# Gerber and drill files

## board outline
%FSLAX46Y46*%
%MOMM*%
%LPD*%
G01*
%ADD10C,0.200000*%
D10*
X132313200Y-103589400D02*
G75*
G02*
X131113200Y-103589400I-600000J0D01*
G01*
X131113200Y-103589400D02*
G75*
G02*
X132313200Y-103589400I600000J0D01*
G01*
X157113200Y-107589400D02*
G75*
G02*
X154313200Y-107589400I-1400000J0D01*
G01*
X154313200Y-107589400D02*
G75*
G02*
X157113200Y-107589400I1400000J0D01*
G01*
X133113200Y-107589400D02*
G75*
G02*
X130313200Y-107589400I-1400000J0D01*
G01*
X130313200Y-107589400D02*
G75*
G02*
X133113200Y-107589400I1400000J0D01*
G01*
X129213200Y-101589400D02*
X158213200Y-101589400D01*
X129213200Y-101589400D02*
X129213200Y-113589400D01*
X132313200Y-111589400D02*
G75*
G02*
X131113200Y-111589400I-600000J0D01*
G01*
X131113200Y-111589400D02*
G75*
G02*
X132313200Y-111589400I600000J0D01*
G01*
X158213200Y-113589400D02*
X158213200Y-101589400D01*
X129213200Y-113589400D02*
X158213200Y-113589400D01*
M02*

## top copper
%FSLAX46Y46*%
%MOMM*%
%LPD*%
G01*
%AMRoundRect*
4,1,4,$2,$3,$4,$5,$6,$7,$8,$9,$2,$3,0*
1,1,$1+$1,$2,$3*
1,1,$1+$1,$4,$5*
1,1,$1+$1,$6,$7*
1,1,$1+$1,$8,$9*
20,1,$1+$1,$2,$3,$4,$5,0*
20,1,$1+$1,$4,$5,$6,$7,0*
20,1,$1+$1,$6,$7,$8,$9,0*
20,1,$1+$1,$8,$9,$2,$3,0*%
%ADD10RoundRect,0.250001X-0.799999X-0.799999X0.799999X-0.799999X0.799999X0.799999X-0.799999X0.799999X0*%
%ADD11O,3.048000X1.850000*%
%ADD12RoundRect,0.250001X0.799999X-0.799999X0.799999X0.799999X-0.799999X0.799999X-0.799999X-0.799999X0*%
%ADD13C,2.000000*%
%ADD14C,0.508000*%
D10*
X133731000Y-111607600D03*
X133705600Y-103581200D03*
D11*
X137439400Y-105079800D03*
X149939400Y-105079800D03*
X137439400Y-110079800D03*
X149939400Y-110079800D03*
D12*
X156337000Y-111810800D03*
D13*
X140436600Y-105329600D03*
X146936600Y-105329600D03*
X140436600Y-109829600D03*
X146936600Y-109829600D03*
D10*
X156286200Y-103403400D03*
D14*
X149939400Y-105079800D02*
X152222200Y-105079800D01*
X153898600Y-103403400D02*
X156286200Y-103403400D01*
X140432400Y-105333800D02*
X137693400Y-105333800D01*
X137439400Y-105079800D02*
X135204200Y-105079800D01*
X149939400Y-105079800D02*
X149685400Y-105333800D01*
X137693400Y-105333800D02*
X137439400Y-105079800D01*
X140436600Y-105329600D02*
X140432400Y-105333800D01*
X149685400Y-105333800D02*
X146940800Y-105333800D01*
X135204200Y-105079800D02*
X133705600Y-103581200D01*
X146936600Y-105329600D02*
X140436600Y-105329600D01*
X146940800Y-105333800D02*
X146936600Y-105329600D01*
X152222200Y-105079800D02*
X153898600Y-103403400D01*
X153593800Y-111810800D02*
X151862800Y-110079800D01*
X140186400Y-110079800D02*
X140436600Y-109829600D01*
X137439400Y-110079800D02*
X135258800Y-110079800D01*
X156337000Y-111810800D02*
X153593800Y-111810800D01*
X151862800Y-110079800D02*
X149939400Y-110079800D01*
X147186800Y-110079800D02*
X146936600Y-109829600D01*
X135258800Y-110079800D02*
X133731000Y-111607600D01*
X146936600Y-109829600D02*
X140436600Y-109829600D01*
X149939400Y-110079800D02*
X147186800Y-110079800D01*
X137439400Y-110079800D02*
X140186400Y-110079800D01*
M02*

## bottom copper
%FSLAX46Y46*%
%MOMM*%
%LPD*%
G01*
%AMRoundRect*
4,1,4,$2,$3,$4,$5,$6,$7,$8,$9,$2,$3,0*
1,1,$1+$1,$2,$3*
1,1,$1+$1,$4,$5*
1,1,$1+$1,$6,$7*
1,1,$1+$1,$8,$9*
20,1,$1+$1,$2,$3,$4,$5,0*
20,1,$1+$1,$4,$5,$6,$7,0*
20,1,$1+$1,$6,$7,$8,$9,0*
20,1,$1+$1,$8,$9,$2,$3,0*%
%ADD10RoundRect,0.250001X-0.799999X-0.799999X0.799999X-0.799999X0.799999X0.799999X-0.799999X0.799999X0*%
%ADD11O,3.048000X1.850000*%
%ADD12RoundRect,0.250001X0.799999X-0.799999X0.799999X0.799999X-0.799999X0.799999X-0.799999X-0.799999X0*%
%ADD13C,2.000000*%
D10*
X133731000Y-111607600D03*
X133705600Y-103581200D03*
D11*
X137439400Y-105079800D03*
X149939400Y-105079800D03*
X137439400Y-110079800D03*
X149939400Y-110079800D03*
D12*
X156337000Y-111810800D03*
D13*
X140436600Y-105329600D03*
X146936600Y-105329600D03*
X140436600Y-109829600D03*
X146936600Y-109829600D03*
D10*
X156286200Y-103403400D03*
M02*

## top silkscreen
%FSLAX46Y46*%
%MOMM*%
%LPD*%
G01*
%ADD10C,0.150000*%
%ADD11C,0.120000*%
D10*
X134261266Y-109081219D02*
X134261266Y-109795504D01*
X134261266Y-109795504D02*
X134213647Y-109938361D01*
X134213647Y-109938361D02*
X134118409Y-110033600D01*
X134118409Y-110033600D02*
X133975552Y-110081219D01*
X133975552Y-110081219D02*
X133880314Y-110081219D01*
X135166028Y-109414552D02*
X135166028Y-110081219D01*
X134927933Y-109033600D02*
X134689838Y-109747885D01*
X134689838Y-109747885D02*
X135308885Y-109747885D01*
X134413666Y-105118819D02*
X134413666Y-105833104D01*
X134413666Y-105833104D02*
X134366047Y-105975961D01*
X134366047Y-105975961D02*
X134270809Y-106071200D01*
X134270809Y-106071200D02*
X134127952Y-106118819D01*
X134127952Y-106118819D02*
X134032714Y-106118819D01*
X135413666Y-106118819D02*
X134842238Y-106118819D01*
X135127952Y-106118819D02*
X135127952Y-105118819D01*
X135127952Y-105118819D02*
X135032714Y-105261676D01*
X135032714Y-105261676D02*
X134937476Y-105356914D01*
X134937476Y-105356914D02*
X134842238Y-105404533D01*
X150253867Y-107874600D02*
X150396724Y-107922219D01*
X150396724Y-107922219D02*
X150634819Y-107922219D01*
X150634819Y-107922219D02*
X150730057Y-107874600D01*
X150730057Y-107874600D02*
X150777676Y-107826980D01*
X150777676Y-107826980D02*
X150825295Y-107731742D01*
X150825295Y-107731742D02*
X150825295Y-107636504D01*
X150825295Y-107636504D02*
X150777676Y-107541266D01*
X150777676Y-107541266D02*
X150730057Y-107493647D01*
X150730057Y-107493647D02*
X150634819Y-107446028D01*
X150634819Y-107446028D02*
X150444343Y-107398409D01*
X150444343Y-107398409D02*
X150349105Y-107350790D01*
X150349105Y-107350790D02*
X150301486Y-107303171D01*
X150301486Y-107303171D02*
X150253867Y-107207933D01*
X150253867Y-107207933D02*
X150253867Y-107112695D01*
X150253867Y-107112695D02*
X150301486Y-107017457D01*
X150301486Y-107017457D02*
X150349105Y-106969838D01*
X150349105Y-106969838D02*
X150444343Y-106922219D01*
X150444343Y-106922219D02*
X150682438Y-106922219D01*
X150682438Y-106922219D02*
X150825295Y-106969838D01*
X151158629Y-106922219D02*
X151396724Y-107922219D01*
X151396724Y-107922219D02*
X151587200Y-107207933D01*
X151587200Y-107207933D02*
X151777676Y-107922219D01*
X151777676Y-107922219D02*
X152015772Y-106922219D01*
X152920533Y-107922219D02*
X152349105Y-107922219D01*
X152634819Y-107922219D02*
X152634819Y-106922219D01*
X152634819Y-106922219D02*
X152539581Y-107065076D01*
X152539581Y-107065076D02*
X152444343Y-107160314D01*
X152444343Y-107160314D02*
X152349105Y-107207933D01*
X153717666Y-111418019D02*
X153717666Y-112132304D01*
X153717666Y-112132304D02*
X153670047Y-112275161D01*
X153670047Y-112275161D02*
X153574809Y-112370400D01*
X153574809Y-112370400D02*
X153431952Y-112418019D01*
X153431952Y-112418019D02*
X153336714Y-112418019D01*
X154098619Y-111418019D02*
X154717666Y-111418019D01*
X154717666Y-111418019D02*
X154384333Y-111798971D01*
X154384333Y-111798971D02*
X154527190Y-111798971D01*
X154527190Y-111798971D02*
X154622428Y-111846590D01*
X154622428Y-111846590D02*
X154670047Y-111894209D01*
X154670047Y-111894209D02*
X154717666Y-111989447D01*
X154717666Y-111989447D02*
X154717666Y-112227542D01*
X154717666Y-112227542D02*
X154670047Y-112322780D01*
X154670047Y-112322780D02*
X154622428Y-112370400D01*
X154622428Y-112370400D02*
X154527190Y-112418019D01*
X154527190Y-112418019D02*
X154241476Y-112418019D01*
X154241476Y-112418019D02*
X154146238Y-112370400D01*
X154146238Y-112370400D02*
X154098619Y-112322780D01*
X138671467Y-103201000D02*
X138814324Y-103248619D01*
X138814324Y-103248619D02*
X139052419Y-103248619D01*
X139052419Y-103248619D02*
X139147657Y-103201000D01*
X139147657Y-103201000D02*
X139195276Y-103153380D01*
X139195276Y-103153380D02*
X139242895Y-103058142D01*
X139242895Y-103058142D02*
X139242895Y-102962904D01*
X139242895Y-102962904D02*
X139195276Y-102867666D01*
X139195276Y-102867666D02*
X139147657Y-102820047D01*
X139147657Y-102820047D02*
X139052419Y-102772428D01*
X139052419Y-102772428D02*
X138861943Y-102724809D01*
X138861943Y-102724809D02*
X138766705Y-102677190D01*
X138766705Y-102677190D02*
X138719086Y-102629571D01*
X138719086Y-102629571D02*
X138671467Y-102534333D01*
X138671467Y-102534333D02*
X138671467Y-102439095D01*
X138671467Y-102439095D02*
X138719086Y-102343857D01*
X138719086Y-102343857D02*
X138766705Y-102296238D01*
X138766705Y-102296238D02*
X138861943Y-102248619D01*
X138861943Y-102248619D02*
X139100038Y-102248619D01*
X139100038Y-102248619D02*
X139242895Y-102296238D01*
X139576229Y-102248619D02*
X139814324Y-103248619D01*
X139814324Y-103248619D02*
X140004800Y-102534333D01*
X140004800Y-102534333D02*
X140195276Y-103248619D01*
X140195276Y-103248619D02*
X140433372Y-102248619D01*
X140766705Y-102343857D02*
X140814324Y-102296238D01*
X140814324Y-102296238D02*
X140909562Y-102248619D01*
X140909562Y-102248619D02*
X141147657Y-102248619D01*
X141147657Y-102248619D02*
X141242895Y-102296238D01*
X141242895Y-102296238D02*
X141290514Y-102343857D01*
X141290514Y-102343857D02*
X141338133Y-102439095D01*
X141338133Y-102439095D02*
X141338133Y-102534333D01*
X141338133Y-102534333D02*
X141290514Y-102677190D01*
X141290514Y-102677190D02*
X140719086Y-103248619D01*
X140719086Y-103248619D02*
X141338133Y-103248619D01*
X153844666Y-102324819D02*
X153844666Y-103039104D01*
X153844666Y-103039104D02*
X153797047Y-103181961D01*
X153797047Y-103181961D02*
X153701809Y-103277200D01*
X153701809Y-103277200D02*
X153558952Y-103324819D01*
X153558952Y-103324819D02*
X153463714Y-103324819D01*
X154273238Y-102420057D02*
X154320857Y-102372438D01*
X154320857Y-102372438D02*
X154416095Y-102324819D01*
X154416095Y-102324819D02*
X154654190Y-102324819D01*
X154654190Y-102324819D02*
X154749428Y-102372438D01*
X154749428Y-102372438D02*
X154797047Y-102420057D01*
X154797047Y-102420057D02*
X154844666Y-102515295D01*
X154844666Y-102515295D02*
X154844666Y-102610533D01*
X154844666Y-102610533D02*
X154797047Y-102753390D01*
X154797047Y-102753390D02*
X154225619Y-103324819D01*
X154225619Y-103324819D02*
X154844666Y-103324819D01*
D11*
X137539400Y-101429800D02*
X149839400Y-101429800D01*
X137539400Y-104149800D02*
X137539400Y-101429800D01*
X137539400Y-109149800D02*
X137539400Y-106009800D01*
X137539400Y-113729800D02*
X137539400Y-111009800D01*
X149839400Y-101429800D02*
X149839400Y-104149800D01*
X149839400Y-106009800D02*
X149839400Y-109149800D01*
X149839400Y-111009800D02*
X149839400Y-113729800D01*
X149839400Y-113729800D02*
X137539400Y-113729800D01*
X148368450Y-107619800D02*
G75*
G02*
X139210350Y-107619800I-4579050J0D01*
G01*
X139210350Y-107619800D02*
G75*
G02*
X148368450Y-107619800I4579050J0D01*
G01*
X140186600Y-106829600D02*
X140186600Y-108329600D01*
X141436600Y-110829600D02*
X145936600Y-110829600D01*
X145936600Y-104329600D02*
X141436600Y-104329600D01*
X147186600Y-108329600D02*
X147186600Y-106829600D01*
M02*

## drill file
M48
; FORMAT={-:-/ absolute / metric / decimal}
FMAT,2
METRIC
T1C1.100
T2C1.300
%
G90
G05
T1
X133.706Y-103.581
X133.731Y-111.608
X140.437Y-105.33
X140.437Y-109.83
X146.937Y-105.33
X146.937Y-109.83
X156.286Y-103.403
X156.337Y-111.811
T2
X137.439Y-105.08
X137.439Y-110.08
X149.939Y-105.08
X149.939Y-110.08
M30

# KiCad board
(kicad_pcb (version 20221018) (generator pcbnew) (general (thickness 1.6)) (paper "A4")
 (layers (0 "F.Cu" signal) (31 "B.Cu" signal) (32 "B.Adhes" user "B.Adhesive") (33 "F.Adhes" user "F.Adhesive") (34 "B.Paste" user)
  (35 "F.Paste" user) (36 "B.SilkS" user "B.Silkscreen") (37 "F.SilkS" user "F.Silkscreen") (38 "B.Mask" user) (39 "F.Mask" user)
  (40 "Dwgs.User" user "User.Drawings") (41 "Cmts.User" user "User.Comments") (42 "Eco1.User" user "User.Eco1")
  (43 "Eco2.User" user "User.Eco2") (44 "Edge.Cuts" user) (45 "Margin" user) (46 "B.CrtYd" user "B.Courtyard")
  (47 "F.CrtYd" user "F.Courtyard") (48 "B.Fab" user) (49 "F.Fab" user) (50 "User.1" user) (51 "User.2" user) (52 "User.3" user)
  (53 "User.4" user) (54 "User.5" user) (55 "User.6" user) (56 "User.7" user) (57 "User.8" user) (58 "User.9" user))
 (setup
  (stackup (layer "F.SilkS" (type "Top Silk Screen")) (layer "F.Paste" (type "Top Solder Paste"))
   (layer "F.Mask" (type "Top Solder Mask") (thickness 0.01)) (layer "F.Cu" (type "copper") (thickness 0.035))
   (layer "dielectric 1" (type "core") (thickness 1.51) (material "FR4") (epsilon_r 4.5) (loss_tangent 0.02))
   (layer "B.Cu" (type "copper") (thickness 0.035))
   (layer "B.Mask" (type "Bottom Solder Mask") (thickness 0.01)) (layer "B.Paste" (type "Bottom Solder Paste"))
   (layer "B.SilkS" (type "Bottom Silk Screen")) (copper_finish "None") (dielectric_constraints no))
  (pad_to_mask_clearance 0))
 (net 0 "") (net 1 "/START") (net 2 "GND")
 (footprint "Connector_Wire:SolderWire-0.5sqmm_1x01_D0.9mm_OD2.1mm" (layer "F.Cu") (at 133.731 111.6076)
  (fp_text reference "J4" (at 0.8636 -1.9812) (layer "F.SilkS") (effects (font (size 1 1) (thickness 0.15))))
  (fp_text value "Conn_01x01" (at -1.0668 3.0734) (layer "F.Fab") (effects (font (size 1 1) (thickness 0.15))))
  (pad "1" thru_hole roundrect (at 0 0) (size 2.1 2.1) (drill 1.1) (layers "*.Cu" "*.Mask") (roundrect_rratio 0.119048) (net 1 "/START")))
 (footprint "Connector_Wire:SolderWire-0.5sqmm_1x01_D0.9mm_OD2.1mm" (layer "F.Cu") (at 133.7056 103.5812)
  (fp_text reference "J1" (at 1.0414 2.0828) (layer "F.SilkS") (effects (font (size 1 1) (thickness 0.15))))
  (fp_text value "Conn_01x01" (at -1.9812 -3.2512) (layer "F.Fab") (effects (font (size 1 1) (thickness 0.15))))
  (pad "1" thru_hole roundrect (at 0 0) (size 2.1 2.1) (drill 1.1) (layers "*.Cu" "*.Mask") (roundrect_rratio 0.119048) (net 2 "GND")))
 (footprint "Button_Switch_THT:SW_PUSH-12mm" (layer "F.Cu") (at 137.4394 105.0798)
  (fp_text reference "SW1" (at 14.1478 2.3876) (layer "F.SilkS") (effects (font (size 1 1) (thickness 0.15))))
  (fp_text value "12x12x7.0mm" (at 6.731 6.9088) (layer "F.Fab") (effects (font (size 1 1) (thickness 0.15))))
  (fp_line (start 0.1 -3.65) (end 12.4 -3.65) (stroke (width 0.12) (type solid)) (layer "F.SilkS"))
  (fp_line (start 0.1 -0.93) (end 0.1 -3.65) (stroke (width 0.12) (type solid)) (layer "F.SilkS"))
  (fp_line (start 0.1 4.07) (end 0.1 0.93) (stroke (width 0.12) (type solid)) (layer "F.SilkS"))
  (fp_line (start 0.1 8.65) (end 0.1 5.93) (stroke (width 0.12) (type solid)) (layer "F.SilkS"))
  (fp_line (start 12.4 -3.65) (end 12.4 -0.93) (stroke (width 0.12) (type solid)) (layer "F.SilkS"))
  (fp_line (start 12.4 0.93) (end 12.4 4.07) (stroke (width 0.12) (type solid)) (layer "F.SilkS"))
  (fp_line (start 12.4 5.93) (end 12.4 8.65) (stroke (width 0.12) (type solid)) (layer "F.SilkS"))
  (fp_line (start 12.4 8.65) (end 0.1 8.65) (stroke (width 0.12) (type solid)) (layer "F.SilkS"))
  (fp_circle (center 6.35 2.54) (end 10.16 5.08) (stroke (width 0.12) (type solid)) (fill none) (layer "F.SilkS"))
  (pad "1" thru_hole oval (at 0 0) (size 3.048 1.85) (drill 1.3) (layers "*.Cu" "*.Mask") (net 2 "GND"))
  (pad "1" thru_hole oval (at 12.5 0) (size 3.048 1.85) (drill 1.3) (layers "*.Cu" "*.Mask") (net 2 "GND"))
  (pad "2" thru_hole oval (at 0 5) (size 3.048 1.85) (drill 1.3) (layers "*.Cu" "*.Mask") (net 1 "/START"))
  (pad "2" thru_hole oval (at 12.5 5) (size 3.048 1.85) (drill 1.3) (layers "*.Cu" "*.Mask") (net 1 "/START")))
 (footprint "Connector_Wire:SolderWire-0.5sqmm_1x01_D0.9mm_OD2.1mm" (layer "F.Cu") (at 156.337 111.8108 90)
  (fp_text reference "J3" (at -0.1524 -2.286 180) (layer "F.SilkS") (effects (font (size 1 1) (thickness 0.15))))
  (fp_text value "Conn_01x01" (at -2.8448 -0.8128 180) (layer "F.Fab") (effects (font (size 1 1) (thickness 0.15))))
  (pad "1" thru_hole roundrect (at 0 0 90) (size 2.1 2.1) (drill 1.1) (layers "*.Cu" "*.Mask") (roundrect_rratio 0.119048) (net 1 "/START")))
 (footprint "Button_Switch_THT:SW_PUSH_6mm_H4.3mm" (layer "F.Cu") (at 140.4366 105.3296)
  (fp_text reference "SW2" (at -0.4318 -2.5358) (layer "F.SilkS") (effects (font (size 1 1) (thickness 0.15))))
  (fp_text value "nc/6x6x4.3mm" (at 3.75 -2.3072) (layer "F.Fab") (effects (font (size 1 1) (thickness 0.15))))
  (fp_line (start -0.25 1.5) (end -0.25 3) (stroke (width 0.12) (type solid)) (layer "F.SilkS"))
  (fp_line (start 1 5.5) (end 5.5 5.5) (stroke (width 0.12) (type solid)) (layer "F.SilkS"))
  (fp_line (start 5.5 -1) (end 1 -1) (stroke (width 0.12) (type solid)) (layer "F.SilkS"))
  (fp_line (start 6.75 3) (end 6.75 1.5) (stroke (width 0.12) (type solid)) (layer "F.SilkS"))
  (pad "1" thru_hole circle (at 0 0 90) (size 2 2) (drill 1.1) (layers "*.Cu" "*.Mask") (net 2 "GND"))
  (pad "1" thru_hole circle (at 6.5 0 90) (size 2 2) (drill 1.1) (layers "*.Cu" "*.Mask") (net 2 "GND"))
  (pad "2" thru_hole circle (at 0 4.5 90) (size 2 2) (drill 1.1) (layers "*.Cu" "*.Mask") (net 1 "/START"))
  (pad "2" thru_hole circle (at 6.5 4.5 90) (size 2 2) (drill 1.1) (layers "*.Cu" "*.Mask") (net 1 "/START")))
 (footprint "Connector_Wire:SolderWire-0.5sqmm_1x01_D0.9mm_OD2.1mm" (layer "F.Cu") (at 156.2862 103.4034)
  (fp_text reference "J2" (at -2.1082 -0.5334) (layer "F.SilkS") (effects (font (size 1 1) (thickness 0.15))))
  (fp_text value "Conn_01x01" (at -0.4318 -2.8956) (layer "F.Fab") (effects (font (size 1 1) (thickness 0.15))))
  (pad "1" thru_hole roundrect (at 0 0) (size 2.1 2.1) (drill 1.1) (layers "*.Cu" "*.Mask") (roundrect_rratio 0.119048) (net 2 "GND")))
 (gr_circle (center 131.7132 103.5894) (end 132.3132 103.5894) (stroke (width 0.2) (type solid)) (fill none) (layer "Edge.Cuts"))
 (gr_circle (center 155.7132 107.5894) (end 157.1132 107.5894) (stroke (width 0.2) (type solid)) (fill none) (layer "Edge.Cuts"))
 (gr_circle (center 131.7132 107.5894) (end 133.1132 107.5894) (stroke (width 0.2) (type solid)) (fill none) (layer "Edge.Cuts"))
 (gr_line (start 129.2132 101.5894) (end 158.2132 101.5894) (stroke (width 0.2) (type solid)) (layer "Edge.Cuts"))
 (gr_line (start 129.2132 101.5894) (end 129.2132 113.5894) (stroke (width 0.2) (type solid)) (layer "Edge.Cuts"))
 (gr_circle (center 131.7132 111.5894) (end 132.3132 111.5894) (stroke (width 0.2) (type solid)) (fill none) (layer "Edge.Cuts"))
 (gr_line (start 158.2132 113.5894) (end 158.2132 101.5894) (stroke (width 0.2) (type solid)) (layer "Edge.Cuts"))
 (gr_line (start 129.2132 113.5894) (end 158.2132 113.5894) (stroke (width 0.2) (type solid)) (layer "Edge.Cuts"))
 (segment (start 149.9394 105.0798) (end 152.2222 105.0798) (width 0.508) (layer "F.Cu") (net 2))
 (segment (start 153.8986 103.4034) (end 156.2862 103.4034) (width 0.508) (layer "F.Cu") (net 2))
 (segment (start 140.4324 105.3338) (end 137.6934 105.3338) (width 0.508) (layer "F.Cu") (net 2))
 (segment (start 137.4394 105.0798) (end 135.2042 105.0798) (width 0.508) (layer "F.Cu") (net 2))
 (segment (start 149.9394 105.0798) (end 149.6854 105.3338) (width 0.508) (layer "F.Cu") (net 2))
 (segment (start 137.6934 105.3338) (end 137.4394 105.0798) (width 0.508) (layer "F.Cu") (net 2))
 (segment (start 140.4366 105.3296) (end 140.4324 105.3338) (width 0.508) (layer "F.Cu") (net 2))
 (segment (start 149.6854 105.3338) (end 146.9408 105.3338) (width 0.508) (layer "F.Cu") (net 2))
 (segment (start 135.2042 105.0798) (end 133.7056 103.5812) (width 0.508) (layer "F.Cu") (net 2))
 (segment (start 146.9366 105.3296) (end 140.4366 105.3296) (width 0.508) (layer "F.Cu") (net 2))
 (segment (start 146.9408 105.3338) (end 146.9366 105.3296) (width 0.508) (layer "F.Cu") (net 2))
 (segment (start 152.2222 105.0798) (end 153.8986 103.4034) (width 0.508) (layer "F.Cu") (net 2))
 (segment (start 153.5938 111.8108) (end 151.8628 110.0798) (width 0.508) (layer "F.Cu") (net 1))
 (segment (start 140.1864 110.0798) (end 140.4366 109.8296) (width 0.508) (layer "F.Cu") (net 1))
 (segment (start 137.4394 110.0798) (end 135.2588 110.0798) (width 0.508) (layer "F.Cu") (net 1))
 (segment (start 156.337 111.8108) (end 153.5938 111.8108) (width 0.508) (layer "F.Cu") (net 1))
 (segment (start 151.8628 110.0798) (end 149.9394 110.0798) (width 0.508) (layer "F.Cu") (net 1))
 (segment (start 147.1868 110.0798) (end 146.9366 109.8296) (width 0.508) (layer "F.Cu") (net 1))
 (segment (start 135.2588 110.0798) (end 133.731 111.6076) (width 0.508) (layer "F.Cu") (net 1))
 (segment (start 146.9366 109.8296) (end 140.4366 109.8296) (width 0.508) (layer "F.Cu") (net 1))
 (segment (start 149.9394 110.0798) (end 147.1868 110.0798) (width 0.508) (layer "F.Cu") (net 1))
 (segment (start 137.4394 110.0798) (end 140.1864 110.0798) (width 0.508) (layer "F.Cu") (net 1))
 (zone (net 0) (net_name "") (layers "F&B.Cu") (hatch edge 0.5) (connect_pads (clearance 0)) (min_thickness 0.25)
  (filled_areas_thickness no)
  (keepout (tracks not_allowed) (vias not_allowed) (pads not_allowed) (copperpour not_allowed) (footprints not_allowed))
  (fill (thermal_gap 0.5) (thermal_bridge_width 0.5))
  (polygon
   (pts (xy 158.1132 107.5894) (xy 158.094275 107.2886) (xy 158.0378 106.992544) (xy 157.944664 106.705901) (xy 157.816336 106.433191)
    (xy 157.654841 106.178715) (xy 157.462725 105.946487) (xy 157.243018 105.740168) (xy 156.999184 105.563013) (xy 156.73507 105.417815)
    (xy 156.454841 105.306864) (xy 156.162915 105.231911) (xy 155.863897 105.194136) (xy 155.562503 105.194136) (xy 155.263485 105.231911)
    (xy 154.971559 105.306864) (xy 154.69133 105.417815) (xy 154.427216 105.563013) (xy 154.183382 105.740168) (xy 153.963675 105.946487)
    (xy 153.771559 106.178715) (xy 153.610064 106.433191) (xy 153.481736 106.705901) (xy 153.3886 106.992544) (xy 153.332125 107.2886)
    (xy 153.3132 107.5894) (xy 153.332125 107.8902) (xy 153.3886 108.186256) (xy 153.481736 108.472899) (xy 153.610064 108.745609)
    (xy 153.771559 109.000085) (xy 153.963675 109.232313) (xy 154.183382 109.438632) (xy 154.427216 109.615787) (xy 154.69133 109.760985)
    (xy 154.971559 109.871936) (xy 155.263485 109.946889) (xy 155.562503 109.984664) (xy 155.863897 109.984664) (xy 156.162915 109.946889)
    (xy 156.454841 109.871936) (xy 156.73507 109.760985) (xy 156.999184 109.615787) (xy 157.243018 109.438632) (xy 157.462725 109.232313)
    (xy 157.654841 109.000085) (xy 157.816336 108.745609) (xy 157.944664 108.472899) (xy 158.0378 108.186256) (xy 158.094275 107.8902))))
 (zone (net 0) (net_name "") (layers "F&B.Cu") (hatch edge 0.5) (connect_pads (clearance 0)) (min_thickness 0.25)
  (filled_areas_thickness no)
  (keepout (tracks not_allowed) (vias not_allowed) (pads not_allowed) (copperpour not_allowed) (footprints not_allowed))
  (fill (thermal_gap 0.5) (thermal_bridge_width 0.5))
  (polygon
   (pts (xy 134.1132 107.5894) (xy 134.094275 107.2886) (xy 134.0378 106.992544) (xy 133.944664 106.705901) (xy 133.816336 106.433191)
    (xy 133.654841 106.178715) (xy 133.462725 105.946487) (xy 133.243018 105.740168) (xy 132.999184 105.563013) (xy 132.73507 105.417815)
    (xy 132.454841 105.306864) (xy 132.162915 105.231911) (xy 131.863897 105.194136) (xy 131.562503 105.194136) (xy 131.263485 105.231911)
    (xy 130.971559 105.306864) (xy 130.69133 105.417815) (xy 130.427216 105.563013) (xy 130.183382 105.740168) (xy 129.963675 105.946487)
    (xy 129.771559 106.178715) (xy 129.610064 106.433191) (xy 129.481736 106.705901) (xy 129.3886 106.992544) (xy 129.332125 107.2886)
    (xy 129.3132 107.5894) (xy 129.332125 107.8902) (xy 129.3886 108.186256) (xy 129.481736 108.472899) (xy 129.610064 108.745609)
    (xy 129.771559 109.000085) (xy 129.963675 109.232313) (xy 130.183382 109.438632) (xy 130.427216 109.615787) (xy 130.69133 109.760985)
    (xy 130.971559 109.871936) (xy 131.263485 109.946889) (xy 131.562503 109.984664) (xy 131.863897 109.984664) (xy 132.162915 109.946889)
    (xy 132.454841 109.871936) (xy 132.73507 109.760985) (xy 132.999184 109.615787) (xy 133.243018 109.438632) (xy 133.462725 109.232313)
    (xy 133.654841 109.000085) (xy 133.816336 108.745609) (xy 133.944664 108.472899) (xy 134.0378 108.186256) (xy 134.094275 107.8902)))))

